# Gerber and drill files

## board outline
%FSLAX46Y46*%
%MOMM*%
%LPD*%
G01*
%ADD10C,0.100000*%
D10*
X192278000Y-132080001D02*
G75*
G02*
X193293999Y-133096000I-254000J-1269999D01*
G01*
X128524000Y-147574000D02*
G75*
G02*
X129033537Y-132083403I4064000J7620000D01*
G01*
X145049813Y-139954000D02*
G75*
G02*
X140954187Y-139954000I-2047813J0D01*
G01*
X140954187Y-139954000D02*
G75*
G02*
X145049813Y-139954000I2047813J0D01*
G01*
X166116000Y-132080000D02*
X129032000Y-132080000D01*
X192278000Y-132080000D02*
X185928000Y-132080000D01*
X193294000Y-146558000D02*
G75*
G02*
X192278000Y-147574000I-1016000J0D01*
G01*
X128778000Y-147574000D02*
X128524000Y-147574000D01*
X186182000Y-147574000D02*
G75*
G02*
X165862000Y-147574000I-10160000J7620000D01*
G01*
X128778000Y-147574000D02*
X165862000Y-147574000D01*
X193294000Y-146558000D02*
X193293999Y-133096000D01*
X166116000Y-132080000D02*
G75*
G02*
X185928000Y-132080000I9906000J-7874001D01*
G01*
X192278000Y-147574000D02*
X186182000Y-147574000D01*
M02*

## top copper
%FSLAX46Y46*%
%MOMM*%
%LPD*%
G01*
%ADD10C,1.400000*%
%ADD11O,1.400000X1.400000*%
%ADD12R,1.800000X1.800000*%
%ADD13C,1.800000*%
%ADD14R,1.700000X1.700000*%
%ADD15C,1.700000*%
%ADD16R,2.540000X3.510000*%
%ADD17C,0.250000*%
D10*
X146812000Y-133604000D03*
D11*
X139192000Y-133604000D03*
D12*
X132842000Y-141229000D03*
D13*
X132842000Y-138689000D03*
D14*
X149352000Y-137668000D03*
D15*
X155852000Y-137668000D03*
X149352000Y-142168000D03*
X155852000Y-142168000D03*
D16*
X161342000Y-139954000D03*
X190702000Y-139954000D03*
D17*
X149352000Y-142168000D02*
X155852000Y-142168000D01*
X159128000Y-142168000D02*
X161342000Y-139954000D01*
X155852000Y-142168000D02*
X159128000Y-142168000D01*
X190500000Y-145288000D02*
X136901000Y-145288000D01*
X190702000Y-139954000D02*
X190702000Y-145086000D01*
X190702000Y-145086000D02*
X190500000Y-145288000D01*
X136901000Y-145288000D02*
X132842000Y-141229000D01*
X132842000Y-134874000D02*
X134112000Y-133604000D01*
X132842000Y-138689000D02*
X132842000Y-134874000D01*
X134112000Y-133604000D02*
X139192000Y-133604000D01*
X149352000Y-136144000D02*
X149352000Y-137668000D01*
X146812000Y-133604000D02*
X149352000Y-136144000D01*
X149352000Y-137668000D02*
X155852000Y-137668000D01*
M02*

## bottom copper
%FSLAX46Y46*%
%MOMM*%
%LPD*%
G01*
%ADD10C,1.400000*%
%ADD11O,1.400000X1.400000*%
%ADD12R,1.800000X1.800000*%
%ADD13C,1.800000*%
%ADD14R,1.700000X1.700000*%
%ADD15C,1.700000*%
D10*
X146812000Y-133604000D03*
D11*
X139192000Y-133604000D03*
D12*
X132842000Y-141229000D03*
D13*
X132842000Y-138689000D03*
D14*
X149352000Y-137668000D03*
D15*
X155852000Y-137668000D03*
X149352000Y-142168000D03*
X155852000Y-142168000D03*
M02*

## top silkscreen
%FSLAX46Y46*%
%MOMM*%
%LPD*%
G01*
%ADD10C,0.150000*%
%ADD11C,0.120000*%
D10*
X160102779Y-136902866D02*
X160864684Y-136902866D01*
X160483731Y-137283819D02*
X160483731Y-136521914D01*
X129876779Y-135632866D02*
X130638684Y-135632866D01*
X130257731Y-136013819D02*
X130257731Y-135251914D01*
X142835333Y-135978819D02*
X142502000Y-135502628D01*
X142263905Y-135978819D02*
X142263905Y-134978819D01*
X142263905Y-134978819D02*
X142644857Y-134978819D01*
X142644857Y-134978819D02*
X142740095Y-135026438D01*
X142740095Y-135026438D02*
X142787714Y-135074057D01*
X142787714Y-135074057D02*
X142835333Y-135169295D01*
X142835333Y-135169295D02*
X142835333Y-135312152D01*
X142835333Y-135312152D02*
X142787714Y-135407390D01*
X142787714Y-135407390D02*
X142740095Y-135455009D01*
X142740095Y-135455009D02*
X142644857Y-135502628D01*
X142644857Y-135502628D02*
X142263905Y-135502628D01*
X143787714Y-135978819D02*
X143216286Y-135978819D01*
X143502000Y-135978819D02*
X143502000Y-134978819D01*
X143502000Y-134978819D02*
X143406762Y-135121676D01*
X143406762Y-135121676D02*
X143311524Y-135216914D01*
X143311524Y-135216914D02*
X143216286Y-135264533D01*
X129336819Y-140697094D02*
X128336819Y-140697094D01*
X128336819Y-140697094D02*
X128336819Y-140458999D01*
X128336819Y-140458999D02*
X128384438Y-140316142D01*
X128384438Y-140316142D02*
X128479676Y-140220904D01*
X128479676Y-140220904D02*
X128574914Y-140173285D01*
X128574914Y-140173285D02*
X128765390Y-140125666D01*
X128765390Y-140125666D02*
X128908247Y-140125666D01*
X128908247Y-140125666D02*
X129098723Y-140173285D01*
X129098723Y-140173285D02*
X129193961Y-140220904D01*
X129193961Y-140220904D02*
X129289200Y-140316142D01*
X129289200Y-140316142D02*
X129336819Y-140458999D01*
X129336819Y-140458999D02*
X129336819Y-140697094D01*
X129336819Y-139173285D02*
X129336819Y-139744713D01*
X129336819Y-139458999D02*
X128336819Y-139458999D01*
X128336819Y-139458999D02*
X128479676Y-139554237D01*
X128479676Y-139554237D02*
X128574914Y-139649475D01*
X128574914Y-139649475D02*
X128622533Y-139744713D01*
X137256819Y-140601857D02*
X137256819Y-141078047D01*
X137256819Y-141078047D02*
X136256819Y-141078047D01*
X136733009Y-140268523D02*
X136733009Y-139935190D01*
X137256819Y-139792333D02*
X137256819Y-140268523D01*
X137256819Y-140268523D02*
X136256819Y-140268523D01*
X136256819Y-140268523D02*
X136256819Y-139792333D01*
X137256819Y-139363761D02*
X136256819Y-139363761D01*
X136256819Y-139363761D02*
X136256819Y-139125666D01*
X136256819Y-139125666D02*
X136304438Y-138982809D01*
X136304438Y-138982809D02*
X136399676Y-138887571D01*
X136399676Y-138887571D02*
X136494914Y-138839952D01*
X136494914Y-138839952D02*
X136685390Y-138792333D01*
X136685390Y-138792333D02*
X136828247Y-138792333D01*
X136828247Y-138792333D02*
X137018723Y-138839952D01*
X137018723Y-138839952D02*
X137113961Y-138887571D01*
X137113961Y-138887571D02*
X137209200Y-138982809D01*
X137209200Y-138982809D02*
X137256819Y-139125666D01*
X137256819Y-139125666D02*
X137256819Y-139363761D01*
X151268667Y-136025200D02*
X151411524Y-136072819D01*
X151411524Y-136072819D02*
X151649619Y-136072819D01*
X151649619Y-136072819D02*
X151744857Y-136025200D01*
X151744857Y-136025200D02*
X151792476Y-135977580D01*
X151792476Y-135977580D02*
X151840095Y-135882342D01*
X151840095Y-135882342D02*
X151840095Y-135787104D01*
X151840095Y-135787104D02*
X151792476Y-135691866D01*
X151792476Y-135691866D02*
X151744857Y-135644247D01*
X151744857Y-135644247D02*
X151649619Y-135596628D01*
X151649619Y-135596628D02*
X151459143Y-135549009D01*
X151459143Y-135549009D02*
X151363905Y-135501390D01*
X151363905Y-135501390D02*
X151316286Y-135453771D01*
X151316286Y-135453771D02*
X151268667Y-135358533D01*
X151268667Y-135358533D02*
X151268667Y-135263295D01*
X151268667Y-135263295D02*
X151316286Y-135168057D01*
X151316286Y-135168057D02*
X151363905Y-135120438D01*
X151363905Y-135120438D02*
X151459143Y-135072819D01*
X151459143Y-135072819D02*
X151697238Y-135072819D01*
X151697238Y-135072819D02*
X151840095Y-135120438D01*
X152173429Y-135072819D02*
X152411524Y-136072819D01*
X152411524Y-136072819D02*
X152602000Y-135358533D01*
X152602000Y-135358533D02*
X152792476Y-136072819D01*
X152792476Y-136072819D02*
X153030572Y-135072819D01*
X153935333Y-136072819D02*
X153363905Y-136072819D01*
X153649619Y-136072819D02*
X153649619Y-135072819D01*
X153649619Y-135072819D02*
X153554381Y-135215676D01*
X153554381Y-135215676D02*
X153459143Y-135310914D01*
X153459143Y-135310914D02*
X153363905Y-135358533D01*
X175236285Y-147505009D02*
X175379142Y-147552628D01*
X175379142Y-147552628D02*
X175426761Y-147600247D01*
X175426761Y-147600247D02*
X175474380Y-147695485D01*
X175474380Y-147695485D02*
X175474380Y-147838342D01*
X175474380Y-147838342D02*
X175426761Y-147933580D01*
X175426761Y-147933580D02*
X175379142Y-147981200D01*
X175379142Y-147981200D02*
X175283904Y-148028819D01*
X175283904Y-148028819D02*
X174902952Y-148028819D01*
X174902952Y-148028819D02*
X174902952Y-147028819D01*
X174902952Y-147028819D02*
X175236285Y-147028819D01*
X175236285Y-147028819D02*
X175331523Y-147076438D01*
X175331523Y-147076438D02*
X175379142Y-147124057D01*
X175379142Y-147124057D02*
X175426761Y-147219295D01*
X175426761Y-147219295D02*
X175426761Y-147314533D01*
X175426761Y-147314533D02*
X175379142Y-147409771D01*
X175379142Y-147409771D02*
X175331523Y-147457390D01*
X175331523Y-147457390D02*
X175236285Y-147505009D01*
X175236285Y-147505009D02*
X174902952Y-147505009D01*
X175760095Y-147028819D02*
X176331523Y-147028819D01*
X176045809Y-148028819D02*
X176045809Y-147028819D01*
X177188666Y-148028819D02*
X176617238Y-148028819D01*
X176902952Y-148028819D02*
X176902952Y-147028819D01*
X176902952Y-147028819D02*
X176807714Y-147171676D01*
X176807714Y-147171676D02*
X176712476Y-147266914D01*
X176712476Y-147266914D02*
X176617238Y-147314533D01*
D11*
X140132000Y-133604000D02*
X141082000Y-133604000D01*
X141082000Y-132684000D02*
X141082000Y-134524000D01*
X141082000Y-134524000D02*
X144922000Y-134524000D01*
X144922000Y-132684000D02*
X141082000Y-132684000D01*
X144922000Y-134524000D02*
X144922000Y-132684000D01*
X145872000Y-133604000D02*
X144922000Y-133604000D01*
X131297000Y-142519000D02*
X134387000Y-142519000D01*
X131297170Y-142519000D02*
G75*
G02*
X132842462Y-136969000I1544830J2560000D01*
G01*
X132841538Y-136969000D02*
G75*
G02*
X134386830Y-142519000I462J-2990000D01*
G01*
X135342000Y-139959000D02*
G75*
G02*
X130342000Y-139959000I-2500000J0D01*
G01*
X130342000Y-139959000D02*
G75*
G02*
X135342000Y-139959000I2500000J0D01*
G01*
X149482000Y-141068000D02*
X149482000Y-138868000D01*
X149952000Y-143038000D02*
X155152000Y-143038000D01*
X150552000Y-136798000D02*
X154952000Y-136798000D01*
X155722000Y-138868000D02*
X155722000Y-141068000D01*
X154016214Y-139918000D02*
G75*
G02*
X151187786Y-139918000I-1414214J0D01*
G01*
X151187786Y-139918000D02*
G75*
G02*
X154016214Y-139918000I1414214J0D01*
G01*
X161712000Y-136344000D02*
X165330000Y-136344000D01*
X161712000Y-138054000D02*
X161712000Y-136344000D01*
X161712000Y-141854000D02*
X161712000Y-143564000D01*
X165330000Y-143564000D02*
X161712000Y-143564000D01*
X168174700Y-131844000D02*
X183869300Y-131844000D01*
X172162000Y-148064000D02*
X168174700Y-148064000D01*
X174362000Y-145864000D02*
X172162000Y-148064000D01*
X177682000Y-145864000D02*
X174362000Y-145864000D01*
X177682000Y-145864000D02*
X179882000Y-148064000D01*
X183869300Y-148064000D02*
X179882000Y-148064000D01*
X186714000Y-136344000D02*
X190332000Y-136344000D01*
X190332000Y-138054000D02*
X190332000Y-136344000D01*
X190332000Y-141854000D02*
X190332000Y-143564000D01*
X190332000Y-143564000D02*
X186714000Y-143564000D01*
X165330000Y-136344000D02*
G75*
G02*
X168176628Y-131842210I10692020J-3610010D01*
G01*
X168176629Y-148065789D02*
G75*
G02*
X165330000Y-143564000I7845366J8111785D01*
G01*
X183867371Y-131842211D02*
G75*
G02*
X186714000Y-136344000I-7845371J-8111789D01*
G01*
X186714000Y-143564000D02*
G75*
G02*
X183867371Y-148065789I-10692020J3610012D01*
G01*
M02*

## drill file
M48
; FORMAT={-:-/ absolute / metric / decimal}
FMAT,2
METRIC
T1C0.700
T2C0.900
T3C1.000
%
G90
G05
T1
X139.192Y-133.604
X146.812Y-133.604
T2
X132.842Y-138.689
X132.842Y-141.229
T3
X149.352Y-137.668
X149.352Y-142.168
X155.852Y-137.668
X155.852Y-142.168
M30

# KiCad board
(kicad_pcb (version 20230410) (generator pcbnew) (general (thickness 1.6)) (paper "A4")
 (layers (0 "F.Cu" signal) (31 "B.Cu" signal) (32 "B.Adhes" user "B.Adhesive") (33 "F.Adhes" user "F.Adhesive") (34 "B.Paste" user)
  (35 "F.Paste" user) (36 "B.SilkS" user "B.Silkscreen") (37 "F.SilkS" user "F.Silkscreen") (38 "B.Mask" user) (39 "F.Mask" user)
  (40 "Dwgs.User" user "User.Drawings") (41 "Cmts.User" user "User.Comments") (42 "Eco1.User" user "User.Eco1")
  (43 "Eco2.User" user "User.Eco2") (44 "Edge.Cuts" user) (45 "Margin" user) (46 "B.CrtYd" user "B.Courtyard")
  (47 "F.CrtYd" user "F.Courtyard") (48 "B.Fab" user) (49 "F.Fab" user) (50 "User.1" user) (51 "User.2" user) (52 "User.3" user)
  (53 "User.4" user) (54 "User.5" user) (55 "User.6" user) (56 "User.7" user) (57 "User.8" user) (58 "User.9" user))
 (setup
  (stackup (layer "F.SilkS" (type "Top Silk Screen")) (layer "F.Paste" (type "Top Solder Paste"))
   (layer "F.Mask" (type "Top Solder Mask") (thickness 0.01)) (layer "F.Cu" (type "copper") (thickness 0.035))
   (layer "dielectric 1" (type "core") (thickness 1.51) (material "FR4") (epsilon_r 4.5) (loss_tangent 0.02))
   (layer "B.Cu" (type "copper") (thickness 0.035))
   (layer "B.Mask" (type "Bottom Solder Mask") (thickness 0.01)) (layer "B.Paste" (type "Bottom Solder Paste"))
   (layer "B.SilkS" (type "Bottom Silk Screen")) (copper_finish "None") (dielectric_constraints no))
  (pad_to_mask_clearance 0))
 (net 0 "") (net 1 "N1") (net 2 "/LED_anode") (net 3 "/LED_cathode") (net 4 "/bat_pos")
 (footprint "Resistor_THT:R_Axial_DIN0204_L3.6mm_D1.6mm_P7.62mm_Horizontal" (layer "F.Cu") (at 146.812 133.604 180)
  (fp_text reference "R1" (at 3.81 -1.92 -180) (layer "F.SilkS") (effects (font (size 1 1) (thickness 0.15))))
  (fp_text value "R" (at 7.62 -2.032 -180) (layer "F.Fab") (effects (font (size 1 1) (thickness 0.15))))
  (fp_line (start 6.68 0) (end 5.73 0) (stroke (width 0.12) (type solid)) (layer "F.SilkS"))
  (fp_line (start 5.73 0.92) (end 5.73 -0.92) (stroke (width 0.12) (type solid)) (layer "F.SilkS"))
  (fp_line (start 5.73 -0.92) (end 1.89 -0.92) (stroke (width 0.12) (type solid)) (layer "F.SilkS"))
  (fp_line (start 1.89 0.92) (end 5.73 0.92) (stroke (width 0.12) (type solid)) (layer "F.SilkS"))
  (fp_line (start 1.89 -0.92) (end 1.89 0.92) (stroke (width 0.12) (type solid)) (layer "F.SilkS"))
  (fp_line (start 0.94 0) (end 1.89 0) (stroke (width 0.12) (type solid)) (layer "F.SilkS"))
  (pad "1" thru_hole circle (at 0 0 180) (size 1.4 1.4) (drill 0.7) (layers "*.Cu" "*.Mask") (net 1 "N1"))
  (pad "2" thru_hole oval (at 7.62 0 180) (size 1.4 1.4) (drill 0.7) (layers "*.Cu" "*.Mask") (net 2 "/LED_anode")))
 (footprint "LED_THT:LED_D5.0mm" (layer "F.Cu") (at 132.842 141.229 90)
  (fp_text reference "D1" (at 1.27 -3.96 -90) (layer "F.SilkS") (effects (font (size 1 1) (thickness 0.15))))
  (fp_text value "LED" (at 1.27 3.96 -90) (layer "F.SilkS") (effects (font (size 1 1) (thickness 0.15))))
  (fp_line (start -1.29 -1.545) (end -1.29 1.545) (stroke (width 0.12) (type solid)) (layer "F.SilkS"))
  (fp_arc (start -1.29 -1.54483) (mid 2.072002 -2.880433) (end 4.26 0.000462) (stroke (width 0.12) (type solid)) (layer "F.SilkS"))
  (fp_arc (start 4.26 -0.000462) (mid 2.072002 2.880433) (end -1.29 1.54483) (stroke (width 0.12) (type solid)) (layer "F.SilkS"))
  (fp_circle (center 1.27 0) (end 3.77 0) (stroke (width 0.12) (type solid)) (fill none) (layer "F.SilkS"))
  (pad "1" thru_hole rect (at 0 0 90) (size 1.8 1.8) (drill 0.9) (layers "*.Cu" "*.Mask") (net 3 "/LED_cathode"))
  (pad "2" thru_hole circle (at 2.54 0 90) (size 1.8 1.8) (drill 0.9) (layers "*.Cu" "*.Mask") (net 2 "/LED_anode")))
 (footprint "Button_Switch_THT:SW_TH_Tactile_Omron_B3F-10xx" (layer "F.Cu") (at 149.352 137.668)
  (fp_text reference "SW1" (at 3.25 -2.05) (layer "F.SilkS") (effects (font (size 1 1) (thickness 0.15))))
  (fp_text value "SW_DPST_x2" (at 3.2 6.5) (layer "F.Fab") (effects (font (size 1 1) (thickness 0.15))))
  (fp_line (start 0.13 3.4) (end 0.13 1.2) (stroke (width 0.12) (type solid)) (layer "F.SilkS"))
  (fp_line (start 0.6 5.37) (end 5.8 5.37) (stroke (width 0.12) (type solid)) (layer "F.SilkS"))
  (fp_line (start 1.2 -0.87) (end 5.6 -0.87) (stroke (width 0.12) (type solid)) (layer "F.SilkS"))
  (fp_line (start 6.37 1.2) (end 6.37 3.4) (stroke (width 0.12) (type solid)) (layer "F.SilkS"))
  (fp_circle (center 3.25 2.25) (end 4.25 3.25) (stroke (width 0.12) (type solid)) (fill none) (layer "F.SilkS"))
  (pad "1" thru_hole rect (at 0 0) (size 1.7 1.7) (drill 1) (layers "*.Cu" "*.Mask") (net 1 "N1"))
  (pad "1" thru_hole circle (at 6.5 0) (size 1.7 1.7) (drill 1) (layers "*.Cu" "*.Mask") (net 1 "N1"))
  (pad "2" thru_hole circle (at 0 4.5) (size 1.7 1.7) (drill 1) (layers "*.Cu" "*.Mask") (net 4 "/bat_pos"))
  (pad "2" thru_hole circle (at 6.5 4.5) (size 1.7 1.7) (drill 1) (layers "*.Cu" "*.Mask") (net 4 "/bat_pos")))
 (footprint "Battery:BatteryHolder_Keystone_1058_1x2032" (layer "F.Cu") (at 176.022 139.954)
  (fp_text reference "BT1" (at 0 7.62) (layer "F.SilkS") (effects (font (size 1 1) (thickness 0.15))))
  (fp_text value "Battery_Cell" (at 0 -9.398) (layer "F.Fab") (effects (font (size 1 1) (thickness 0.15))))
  (fp_line (start -14.31 -3.61) (end -10.692 -3.61) (stroke (width 0.12) (type solid)) (layer "F.SilkS"))
  (fp_line (start -14.31 -1.9) (end -14.31 -3.61) (stroke (width 0.12) (type solid)) (layer "F.SilkS"))
  (fp_line (start -14.31 1.9) (end -14.31 3.61) (stroke (width 0.12) (type solid)) (layer "F.SilkS"))
  (fp_line (start -10.692 3.61) (end -14.31 3.61) (stroke (width 0.12) (type solid)) (layer "F.SilkS"))
  (fp_line (start -7.8473 -8.11) (end 7.8473 -8.11) (stroke (width 0.12) (type solid)) (layer "F.SilkS"))
  (fp_line (start -3.86 8.11) (end -7.8473 8.11) (stroke (width 0.12) (type solid)) (layer "F.SilkS"))
  (fp_line (start -1.66 5.91) (end -3.86 8.11) (stroke (width 0.12) (type solid)) (layer "F.SilkS"))
  (fp_line (start 1.66 5.91) (end -1.66 5.91) (stroke (width 0.12) (type solid)) (layer "F.SilkS"))
  (fp_line (start 1.66 5.91) (end 3.86 8.11) (stroke (width 0.12) (type solid)) (layer "F.SilkS"))
  (fp_line (start 7.8473 8.11) (end 3.86 8.11) (stroke (width 0.12) (type solid)) (layer "F.SilkS"))
  (fp_line (start 10.692 -3.61) (end 14.31 -3.61) (stroke (width 0.12) (type solid)) (layer "F.SilkS"))
  (fp_line (start 14.31 -1.9) (end 14.31 -3.61) (stroke (width 0.12) (type solid)) (layer "F.SilkS"))
  (fp_line (start 14.31 1.9) (end 14.31 3.61) (stroke (width 0.12) (type solid)) (layer "F.SilkS"))
  (fp_line (start 14.31 3.61) (end 10.692 3.61) (stroke (width 0.12) (type solid)) (layer "F.SilkS"))
  (fp_arc (start -10.692 -3.61) (mid -9.538084 -6.031244) (end -7.845371 -8.111789) (stroke (width 0.12) (type solid)) (layer "F.SilkS"))
  (fp_arc (start -7.845371 8.111789) (mid -9.538085 6.031244) (end -10.692 3.61) (stroke (width 0.12) (type solid)) (layer "F.SilkS"))
  (fp_arc (start 7.845371 -8.111789) (mid 9.538085 -6.031244) (end 10.692 -3.61) (stroke (width 0.12) (type solid)) (layer "F.SilkS"))
  (fp_arc (start 10.692 3.61) (mid 9.538084 6.031244) (end 7.845371 8.111789) (stroke (width 0.12) (type solid)) (layer "F.SilkS"))
  (pad "1" smd rect (at -14.68 0) (size 2.54 3.51) (layers "F.Cu" "F.Paste" "F.Mask") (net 4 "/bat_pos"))
  (pad "2" smd rect (at 14.68 0) (size 2.54 3.51) (layers "F.Cu" "F.Paste" "F.Mask") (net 3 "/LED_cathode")))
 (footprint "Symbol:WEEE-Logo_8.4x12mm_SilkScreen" (layer "B.Cu") (at 176.022 139.954 180)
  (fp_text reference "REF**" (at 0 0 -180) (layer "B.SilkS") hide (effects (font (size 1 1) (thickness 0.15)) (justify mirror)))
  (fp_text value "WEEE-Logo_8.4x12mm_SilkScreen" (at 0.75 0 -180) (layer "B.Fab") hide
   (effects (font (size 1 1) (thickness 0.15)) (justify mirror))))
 (gr_arc (start 192.278 132.080001) (mid 192.939809 132.434191) (end 193.293999 133.096) (stroke (width 0.1) (type default))
  (layer "Edge.Cuts"))
 (gr_arc (start 128.524 147.574) (mid 123.956668 139.670087) (end 129.033537 132.083403) (stroke (width 0.1) (type default))
  (layer "Edge.Cuts"))
 (gr_circle (center 143.002 139.954) (end 144.018 141.732) (stroke (width 0.1) (type default)) (fill none) (layer "Edge.Cuts"))
 (gr_line (start 166.116 132.08) (end 129.032 132.08) (stroke (width 0.1) (type default)) (layer "Edge.Cuts"))
 (gr_line (start 192.278 132.08) (end 185.928 132.08) (stroke (width 0.1) (type default)) (layer "Edge.Cuts"))
 (gr_arc (start 193.294 146.558) (mid 192.99642 147.27642) (end 192.278 147.574) (stroke (width 0.1) (type default)) (layer "Edge.Cuts"))
 (gr_line (start 128.778 147.574) (end 128.524 147.574) (stroke (width 0.1) (type default)) (layer "Edge.Cuts"))
 (gr_arc (start 186.182 147.574) (mid 176.022 152.654) (end 165.862 147.574) (stroke (width 0.1) (type default)) (layer "Edge.Cuts"))
 (gr_line (start 128.778 147.574) (end 165.862 147.574) (stroke (width 0.1) (type default)) (layer "Edge.Cuts"))
 (gr_line (start 193.294 146.558) (end 193.293999 133.096) (stroke (width 0.1) (type default)) (layer "Edge.Cuts"))
 (gr_arc (start 166.116 132.08) (mid 176.022 127.299803) (end 185.928 132.08) (stroke (width 0.1) (type default)) (layer "Edge.Cuts"))
 (gr_line (start 192.278 147.574) (end 186.182 147.574) (stroke (width 0.1) (type default)) (layer "Edge.Cuts"))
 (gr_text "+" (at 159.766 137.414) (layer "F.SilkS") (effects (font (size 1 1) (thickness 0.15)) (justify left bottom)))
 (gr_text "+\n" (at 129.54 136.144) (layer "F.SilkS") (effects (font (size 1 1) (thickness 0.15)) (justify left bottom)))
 (segment (start 149.352 142.168) (end 155.852 142.168) (width 0.25) (layer "F.Cu") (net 4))
 (segment (start 159.128 142.168) (end 161.342 139.954) (width 0.25) (layer "F.Cu") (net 4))
 (segment (start 155.852 142.168) (end 159.128 142.168) (width 0.25) (layer "F.Cu") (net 4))
 (segment (start 190.5 145.288) (end 136.901 145.288) (width 0.25) (layer "F.Cu") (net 3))
 (segment (start 190.702 139.954) (end 190.702 145.086) (width 0.25) (layer "F.Cu") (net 3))
 (segment (start 190.702 145.086) (end 190.5 145.288) (width 0.25) (layer "F.Cu") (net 3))
 (segment (start 136.901 145.288) (end 132.842 141.229) (width 0.25) (layer "F.Cu") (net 3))
 (segment (start 132.842 134.874) (end 134.112 133.604) (width 0.25) (layer "F.Cu") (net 2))
 (segment (start 132.842 138.689) (end 132.842 134.874) (width 0.25) (layer "F.Cu") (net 2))
 (segment (start 134.112 133.604) (end 139.192 133.604) (width 0.25) (layer "F.Cu") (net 2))
 (segment (start 149.352 136.144) (end 149.352 137.668) (width 0.25) (layer "F.Cu") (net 1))
 (segment (start 146.812 133.604) (end 149.352 136.144) (width 0.25) (layer "F.Cu") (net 1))
 (segment (start 149.352 137.668) (end 155.852 137.668) (width 0.25) (layer "F.Cu") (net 1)))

